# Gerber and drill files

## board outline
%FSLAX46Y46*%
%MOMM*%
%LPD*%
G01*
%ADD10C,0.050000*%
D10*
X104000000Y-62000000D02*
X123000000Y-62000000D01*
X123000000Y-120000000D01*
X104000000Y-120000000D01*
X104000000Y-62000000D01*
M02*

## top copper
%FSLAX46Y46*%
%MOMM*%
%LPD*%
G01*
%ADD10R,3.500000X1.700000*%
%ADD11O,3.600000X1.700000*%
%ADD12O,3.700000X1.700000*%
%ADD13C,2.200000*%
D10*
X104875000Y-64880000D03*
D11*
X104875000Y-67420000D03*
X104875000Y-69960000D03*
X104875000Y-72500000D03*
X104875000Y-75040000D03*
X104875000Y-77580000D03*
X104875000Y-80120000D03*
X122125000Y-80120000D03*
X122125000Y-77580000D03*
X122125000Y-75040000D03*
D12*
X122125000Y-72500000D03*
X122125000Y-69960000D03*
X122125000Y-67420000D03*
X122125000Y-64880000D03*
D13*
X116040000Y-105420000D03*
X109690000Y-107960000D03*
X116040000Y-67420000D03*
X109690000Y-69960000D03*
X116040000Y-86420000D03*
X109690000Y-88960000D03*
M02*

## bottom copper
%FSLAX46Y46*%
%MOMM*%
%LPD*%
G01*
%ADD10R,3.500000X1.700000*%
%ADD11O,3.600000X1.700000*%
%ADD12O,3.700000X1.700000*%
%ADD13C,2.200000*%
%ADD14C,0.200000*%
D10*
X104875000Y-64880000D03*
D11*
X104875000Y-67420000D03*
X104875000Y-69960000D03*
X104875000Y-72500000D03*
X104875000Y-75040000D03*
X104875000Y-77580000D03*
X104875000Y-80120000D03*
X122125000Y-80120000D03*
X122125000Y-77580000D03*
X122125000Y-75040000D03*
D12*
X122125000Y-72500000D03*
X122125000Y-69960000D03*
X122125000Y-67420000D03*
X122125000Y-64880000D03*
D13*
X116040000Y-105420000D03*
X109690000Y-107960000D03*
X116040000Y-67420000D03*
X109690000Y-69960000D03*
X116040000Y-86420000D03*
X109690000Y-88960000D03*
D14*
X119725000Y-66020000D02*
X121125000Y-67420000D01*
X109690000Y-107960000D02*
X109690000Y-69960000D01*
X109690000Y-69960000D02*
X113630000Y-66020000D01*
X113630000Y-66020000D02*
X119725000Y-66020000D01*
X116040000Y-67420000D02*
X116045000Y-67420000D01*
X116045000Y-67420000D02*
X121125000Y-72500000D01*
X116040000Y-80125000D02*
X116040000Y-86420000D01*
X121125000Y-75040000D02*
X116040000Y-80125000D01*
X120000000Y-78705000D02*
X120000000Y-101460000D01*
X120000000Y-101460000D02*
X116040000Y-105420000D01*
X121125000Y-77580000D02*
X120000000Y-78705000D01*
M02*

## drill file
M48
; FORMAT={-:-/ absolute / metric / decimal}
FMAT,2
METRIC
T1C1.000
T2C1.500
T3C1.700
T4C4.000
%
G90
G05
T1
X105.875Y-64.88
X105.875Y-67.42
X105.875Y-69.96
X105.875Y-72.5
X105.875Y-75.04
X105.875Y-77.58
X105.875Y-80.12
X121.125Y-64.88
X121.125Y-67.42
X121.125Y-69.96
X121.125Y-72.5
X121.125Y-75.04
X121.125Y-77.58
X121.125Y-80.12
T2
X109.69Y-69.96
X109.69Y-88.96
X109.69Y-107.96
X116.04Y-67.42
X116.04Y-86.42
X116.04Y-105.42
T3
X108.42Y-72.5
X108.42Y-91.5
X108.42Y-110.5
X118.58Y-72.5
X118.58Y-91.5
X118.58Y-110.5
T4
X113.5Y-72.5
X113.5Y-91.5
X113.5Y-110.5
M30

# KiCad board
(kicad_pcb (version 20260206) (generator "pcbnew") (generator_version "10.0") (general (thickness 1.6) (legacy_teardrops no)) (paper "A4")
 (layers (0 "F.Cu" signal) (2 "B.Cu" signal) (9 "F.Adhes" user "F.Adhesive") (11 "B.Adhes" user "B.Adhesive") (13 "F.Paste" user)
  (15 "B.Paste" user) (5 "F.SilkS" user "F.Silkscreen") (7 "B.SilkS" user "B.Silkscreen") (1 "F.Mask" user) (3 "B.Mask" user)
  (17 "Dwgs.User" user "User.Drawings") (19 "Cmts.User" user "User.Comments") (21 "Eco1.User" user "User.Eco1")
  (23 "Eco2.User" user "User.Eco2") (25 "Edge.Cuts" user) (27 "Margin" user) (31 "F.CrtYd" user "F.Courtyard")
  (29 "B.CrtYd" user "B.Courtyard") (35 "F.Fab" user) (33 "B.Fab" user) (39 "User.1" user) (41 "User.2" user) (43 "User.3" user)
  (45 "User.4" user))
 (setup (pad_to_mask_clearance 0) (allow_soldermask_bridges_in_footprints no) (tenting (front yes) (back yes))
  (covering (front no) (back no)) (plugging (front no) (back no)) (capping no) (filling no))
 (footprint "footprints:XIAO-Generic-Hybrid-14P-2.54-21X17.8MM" (layer "F.Cu") (at 113.5 72.5)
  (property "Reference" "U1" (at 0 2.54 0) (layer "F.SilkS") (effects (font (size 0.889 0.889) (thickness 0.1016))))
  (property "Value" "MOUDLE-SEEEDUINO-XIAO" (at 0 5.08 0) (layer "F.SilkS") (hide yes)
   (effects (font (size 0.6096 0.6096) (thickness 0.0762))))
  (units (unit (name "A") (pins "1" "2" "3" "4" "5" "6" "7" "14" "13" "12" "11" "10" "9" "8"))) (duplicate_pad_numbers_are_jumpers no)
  (pad "1" thru_hole rect (at -7.625 -7.62) (size 3.5 1.7) (drill 1 (offset -1 0)) (layers "*.Cu" "*.Mask") (remove_unused_layers no)
   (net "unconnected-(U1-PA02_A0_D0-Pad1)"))
  (pad "2" thru_hole oval (at -7.625 -5.08) (size 3.6 1.7) (drill 1 (offset -1 0)) (layers "*.Cu" "*.Mask") (remove_unused_layers no)
   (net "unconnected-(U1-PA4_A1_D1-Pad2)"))
  (pad "3" thru_hole oval (at -7.625 -2.54) (size 3.6 1.7) (drill 1 (offset -1 0)) (layers "*.Cu" "*.Mask") (remove_unused_layers no)
   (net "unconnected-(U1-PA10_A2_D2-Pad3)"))
  (pad "4" thru_hole oval (at -7.625 0) (size 3.6 1.7) (drill 1 (offset -1 0)) (layers "*.Cu" "*.Mask") (remove_unused_layers no)
   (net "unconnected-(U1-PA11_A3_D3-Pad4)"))
  (pad "5" thru_hole oval (at -7.625 2.54) (size 3.6 1.7) (drill 1 (offset -1 0)) (layers "*.Cu" "*.Mask") (remove_unused_layers no)
   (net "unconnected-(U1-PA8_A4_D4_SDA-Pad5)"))
  (pad "6" thru_hole oval (at -7.625 5.08 180) (size 3.6 1.7) (drill 1 (offset 1 0)) (layers "*.Cu" "*.Mask") (remove_unused_layers no)
   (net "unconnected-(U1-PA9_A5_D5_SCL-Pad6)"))
  (pad "7" thru_hole oval (at -7.625 7.62) (size 3.6 1.7) (drill 1 (offset -1 0)) (layers "*.Cu" "*.Mask") (remove_unused_layers no)
   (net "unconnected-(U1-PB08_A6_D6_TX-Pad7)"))
  (pad "8" thru_hole oval (at 7.625 7.62) (size 3.6 1.7) (drill 1 (offset 1 0)) (layers "*.Cu" "*.Mask") (remove_unused_layers no)
   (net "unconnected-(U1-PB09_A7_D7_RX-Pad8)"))
  (pad "9" thru_hole oval (at 7.625 5.08) (size 3.6 1.7) (drill 1 (offset 1 0)) (layers "*.Cu" "*.Mask") (remove_unused_layers no)
   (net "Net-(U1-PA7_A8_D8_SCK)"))
  (pad "10" thru_hole oval (at 7.625 2.54) (size 3.6 1.7) (drill 1 (offset 1 0)) (layers "*.Cu" "*.Mask") (remove_unused_layers no)
   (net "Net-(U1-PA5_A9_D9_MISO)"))
  (pad "11" thru_hole oval (at 7.625 0) (size 3.7 1.7) (drill 1 (offset 1 0)) (layers "*.Cu" "*.Mask") (remove_unused_layers no)
   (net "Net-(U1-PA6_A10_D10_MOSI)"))
  (pad "12" thru_hole oval (at 7.625 -2.54) (size 3.7 1.7) (drill 1 (offset 1 0)) (layers "*.Cu" "*.Mask") (remove_unused_layers no)
   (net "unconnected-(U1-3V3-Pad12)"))
  (pad "13" thru_hole oval (at 7.625 -5.08) (size 3.7 1.7) (drill 1 (offset 1 0)) (layers "*.Cu" "*.Mask") (remove_unused_layers no)
   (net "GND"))
  (pad "14" thru_hole oval (at 7.625 -7.62) (size 3.7 1.7) (drill 1 (offset 1 0)) (layers "*.Cu" "*.Mask") (remove_unused_layers no)
   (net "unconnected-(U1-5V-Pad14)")))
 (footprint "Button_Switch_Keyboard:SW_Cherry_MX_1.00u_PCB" (layer "F.Cu") (at 116.04 105.42)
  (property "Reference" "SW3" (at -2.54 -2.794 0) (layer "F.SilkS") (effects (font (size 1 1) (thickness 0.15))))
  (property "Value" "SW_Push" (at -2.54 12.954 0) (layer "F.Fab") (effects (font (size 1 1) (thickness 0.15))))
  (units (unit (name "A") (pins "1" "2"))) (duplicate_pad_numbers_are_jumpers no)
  (pad "" np_thru_hole circle (at -7.62 5.08) (size 1.7 1.7) (drill 1.7) (layers "*.Cu" "*.Mask"))
  (pad "" np_thru_hole circle (at -2.54 5.08) (size 4 4) (drill 4) (layers "*.Cu" "*.Mask"))
  (pad "" np_thru_hole circle (at 2.54 5.08) (size 1.7 1.7) (drill 1.7) (layers "*.Cu" "*.Mask"))
  (pad "1" thru_hole circle (at 0 0) (size 2.2 2.2) (drill 1.5) (layers "*.Cu" "*.Mask") (remove_unused_layers no)
   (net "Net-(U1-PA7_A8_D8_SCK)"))
  (pad "2" thru_hole circle (at -6.35 2.54) (size 2.2 2.2) (drill 1.5) (layers "*.Cu" "*.Mask") (remove_unused_layers no) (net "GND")))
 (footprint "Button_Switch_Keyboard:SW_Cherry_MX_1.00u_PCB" (layer "F.Cu") (at 116.04 67.42)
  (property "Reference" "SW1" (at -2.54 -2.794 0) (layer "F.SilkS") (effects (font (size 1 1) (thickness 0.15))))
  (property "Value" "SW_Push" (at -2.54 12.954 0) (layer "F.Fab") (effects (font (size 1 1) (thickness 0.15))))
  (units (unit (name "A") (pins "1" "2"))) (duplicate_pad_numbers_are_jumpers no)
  (pad "" np_thru_hole circle (at -7.62 5.08) (size 1.7 1.7) (drill 1.7) (layers "*.Cu" "*.Mask"))
  (pad "" np_thru_hole circle (at -2.54 5.08) (size 4 4) (drill 4) (layers "*.Cu" "*.Mask"))
  (pad "" np_thru_hole circle (at 2.54 5.08) (size 1.7 1.7) (drill 1.7) (layers "*.Cu" "*.Mask"))
  (pad "1" thru_hole circle (at 0 0) (size 2.2 2.2) (drill 1.5) (layers "*.Cu" "*.Mask") (remove_unused_layers no)
   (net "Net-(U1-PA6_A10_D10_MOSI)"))
  (pad "2" thru_hole circle (at -6.35 2.54) (size 2.2 2.2) (drill 1.5) (layers "*.Cu" "*.Mask") (remove_unused_layers no) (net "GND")))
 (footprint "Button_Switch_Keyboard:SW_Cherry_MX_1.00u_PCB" (layer "F.Cu") (at 116.04 86.42)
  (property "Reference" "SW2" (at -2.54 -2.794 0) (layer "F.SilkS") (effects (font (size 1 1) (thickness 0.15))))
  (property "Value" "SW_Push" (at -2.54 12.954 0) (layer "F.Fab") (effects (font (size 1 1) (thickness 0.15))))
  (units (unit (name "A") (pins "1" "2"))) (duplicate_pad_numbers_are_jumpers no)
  (pad "" np_thru_hole circle (at -7.62 5.08) (size 1.7 1.7) (drill 1.7) (layers "*.Cu" "*.Mask"))
  (pad "" np_thru_hole circle (at -2.54 5.08) (size 4 4) (drill 4) (layers "*.Cu" "*.Mask"))
  (pad "" np_thru_hole circle (at 2.54 5.08) (size 1.7 1.7) (drill 1.7) (layers "*.Cu" "*.Mask"))
  (pad "1" thru_hole circle (at 0 0) (size 2.2 2.2) (drill 1.5) (layers "*.Cu" "*.Mask") (remove_unused_layers no)
   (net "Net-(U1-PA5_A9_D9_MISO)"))
  (pad "2" thru_hole circle (at -6.35 2.54) (size 2.2 2.2) (drill 1.5) (layers "*.Cu" "*.Mask") (remove_unused_layers no) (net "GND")))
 (gr_rect (start 104 62) (end 123 120) (stroke (width 0.05) (type default)) (fill no) (layer "Edge.Cuts"))
 (segment (start 119.725 66.02) (end 121.125 67.42) (width 0.2) (layer "B.Cu") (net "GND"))
 (segment (start 109.69 107.96) (end 109.69 69.96) (width 0.2) (layer "B.Cu") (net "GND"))
 (segment (start 109.69 69.96) (end 113.63 66.02) (width 0.2) (layer "B.Cu") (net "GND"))
 (segment (start 113.63 66.02) (end 119.725 66.02) (width 0.2) (layer "B.Cu") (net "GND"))
 (segment (start 116.04 67.42) (end 116.045 67.42) (width 0.2) (layer "B.Cu") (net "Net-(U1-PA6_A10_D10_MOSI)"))
 (segment (start 116.045 67.42) (end 121.125 72.5) (width 0.2) (layer "B.Cu") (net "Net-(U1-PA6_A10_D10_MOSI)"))
 (segment (start 116.04 80.125) (end 116.04 86.42) (width 0.2) (layer "B.Cu") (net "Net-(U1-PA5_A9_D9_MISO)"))
 (segment (start 121.125 75.04) (end 116.04 80.125) (width 0.2) (layer "B.Cu") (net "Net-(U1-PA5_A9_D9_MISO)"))
 (segment (start 120 78.705) (end 120 101.46) (width 0.2) (layer "B.Cu") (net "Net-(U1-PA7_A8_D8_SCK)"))
 (segment (start 120 101.46) (end 116.04 105.42) (width 0.2) (layer "B.Cu") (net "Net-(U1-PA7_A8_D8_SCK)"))
 (segment (start 121.125 77.58) (end 120 78.705) (width 0.2) (layer "B.Cu") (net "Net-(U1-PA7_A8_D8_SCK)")))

